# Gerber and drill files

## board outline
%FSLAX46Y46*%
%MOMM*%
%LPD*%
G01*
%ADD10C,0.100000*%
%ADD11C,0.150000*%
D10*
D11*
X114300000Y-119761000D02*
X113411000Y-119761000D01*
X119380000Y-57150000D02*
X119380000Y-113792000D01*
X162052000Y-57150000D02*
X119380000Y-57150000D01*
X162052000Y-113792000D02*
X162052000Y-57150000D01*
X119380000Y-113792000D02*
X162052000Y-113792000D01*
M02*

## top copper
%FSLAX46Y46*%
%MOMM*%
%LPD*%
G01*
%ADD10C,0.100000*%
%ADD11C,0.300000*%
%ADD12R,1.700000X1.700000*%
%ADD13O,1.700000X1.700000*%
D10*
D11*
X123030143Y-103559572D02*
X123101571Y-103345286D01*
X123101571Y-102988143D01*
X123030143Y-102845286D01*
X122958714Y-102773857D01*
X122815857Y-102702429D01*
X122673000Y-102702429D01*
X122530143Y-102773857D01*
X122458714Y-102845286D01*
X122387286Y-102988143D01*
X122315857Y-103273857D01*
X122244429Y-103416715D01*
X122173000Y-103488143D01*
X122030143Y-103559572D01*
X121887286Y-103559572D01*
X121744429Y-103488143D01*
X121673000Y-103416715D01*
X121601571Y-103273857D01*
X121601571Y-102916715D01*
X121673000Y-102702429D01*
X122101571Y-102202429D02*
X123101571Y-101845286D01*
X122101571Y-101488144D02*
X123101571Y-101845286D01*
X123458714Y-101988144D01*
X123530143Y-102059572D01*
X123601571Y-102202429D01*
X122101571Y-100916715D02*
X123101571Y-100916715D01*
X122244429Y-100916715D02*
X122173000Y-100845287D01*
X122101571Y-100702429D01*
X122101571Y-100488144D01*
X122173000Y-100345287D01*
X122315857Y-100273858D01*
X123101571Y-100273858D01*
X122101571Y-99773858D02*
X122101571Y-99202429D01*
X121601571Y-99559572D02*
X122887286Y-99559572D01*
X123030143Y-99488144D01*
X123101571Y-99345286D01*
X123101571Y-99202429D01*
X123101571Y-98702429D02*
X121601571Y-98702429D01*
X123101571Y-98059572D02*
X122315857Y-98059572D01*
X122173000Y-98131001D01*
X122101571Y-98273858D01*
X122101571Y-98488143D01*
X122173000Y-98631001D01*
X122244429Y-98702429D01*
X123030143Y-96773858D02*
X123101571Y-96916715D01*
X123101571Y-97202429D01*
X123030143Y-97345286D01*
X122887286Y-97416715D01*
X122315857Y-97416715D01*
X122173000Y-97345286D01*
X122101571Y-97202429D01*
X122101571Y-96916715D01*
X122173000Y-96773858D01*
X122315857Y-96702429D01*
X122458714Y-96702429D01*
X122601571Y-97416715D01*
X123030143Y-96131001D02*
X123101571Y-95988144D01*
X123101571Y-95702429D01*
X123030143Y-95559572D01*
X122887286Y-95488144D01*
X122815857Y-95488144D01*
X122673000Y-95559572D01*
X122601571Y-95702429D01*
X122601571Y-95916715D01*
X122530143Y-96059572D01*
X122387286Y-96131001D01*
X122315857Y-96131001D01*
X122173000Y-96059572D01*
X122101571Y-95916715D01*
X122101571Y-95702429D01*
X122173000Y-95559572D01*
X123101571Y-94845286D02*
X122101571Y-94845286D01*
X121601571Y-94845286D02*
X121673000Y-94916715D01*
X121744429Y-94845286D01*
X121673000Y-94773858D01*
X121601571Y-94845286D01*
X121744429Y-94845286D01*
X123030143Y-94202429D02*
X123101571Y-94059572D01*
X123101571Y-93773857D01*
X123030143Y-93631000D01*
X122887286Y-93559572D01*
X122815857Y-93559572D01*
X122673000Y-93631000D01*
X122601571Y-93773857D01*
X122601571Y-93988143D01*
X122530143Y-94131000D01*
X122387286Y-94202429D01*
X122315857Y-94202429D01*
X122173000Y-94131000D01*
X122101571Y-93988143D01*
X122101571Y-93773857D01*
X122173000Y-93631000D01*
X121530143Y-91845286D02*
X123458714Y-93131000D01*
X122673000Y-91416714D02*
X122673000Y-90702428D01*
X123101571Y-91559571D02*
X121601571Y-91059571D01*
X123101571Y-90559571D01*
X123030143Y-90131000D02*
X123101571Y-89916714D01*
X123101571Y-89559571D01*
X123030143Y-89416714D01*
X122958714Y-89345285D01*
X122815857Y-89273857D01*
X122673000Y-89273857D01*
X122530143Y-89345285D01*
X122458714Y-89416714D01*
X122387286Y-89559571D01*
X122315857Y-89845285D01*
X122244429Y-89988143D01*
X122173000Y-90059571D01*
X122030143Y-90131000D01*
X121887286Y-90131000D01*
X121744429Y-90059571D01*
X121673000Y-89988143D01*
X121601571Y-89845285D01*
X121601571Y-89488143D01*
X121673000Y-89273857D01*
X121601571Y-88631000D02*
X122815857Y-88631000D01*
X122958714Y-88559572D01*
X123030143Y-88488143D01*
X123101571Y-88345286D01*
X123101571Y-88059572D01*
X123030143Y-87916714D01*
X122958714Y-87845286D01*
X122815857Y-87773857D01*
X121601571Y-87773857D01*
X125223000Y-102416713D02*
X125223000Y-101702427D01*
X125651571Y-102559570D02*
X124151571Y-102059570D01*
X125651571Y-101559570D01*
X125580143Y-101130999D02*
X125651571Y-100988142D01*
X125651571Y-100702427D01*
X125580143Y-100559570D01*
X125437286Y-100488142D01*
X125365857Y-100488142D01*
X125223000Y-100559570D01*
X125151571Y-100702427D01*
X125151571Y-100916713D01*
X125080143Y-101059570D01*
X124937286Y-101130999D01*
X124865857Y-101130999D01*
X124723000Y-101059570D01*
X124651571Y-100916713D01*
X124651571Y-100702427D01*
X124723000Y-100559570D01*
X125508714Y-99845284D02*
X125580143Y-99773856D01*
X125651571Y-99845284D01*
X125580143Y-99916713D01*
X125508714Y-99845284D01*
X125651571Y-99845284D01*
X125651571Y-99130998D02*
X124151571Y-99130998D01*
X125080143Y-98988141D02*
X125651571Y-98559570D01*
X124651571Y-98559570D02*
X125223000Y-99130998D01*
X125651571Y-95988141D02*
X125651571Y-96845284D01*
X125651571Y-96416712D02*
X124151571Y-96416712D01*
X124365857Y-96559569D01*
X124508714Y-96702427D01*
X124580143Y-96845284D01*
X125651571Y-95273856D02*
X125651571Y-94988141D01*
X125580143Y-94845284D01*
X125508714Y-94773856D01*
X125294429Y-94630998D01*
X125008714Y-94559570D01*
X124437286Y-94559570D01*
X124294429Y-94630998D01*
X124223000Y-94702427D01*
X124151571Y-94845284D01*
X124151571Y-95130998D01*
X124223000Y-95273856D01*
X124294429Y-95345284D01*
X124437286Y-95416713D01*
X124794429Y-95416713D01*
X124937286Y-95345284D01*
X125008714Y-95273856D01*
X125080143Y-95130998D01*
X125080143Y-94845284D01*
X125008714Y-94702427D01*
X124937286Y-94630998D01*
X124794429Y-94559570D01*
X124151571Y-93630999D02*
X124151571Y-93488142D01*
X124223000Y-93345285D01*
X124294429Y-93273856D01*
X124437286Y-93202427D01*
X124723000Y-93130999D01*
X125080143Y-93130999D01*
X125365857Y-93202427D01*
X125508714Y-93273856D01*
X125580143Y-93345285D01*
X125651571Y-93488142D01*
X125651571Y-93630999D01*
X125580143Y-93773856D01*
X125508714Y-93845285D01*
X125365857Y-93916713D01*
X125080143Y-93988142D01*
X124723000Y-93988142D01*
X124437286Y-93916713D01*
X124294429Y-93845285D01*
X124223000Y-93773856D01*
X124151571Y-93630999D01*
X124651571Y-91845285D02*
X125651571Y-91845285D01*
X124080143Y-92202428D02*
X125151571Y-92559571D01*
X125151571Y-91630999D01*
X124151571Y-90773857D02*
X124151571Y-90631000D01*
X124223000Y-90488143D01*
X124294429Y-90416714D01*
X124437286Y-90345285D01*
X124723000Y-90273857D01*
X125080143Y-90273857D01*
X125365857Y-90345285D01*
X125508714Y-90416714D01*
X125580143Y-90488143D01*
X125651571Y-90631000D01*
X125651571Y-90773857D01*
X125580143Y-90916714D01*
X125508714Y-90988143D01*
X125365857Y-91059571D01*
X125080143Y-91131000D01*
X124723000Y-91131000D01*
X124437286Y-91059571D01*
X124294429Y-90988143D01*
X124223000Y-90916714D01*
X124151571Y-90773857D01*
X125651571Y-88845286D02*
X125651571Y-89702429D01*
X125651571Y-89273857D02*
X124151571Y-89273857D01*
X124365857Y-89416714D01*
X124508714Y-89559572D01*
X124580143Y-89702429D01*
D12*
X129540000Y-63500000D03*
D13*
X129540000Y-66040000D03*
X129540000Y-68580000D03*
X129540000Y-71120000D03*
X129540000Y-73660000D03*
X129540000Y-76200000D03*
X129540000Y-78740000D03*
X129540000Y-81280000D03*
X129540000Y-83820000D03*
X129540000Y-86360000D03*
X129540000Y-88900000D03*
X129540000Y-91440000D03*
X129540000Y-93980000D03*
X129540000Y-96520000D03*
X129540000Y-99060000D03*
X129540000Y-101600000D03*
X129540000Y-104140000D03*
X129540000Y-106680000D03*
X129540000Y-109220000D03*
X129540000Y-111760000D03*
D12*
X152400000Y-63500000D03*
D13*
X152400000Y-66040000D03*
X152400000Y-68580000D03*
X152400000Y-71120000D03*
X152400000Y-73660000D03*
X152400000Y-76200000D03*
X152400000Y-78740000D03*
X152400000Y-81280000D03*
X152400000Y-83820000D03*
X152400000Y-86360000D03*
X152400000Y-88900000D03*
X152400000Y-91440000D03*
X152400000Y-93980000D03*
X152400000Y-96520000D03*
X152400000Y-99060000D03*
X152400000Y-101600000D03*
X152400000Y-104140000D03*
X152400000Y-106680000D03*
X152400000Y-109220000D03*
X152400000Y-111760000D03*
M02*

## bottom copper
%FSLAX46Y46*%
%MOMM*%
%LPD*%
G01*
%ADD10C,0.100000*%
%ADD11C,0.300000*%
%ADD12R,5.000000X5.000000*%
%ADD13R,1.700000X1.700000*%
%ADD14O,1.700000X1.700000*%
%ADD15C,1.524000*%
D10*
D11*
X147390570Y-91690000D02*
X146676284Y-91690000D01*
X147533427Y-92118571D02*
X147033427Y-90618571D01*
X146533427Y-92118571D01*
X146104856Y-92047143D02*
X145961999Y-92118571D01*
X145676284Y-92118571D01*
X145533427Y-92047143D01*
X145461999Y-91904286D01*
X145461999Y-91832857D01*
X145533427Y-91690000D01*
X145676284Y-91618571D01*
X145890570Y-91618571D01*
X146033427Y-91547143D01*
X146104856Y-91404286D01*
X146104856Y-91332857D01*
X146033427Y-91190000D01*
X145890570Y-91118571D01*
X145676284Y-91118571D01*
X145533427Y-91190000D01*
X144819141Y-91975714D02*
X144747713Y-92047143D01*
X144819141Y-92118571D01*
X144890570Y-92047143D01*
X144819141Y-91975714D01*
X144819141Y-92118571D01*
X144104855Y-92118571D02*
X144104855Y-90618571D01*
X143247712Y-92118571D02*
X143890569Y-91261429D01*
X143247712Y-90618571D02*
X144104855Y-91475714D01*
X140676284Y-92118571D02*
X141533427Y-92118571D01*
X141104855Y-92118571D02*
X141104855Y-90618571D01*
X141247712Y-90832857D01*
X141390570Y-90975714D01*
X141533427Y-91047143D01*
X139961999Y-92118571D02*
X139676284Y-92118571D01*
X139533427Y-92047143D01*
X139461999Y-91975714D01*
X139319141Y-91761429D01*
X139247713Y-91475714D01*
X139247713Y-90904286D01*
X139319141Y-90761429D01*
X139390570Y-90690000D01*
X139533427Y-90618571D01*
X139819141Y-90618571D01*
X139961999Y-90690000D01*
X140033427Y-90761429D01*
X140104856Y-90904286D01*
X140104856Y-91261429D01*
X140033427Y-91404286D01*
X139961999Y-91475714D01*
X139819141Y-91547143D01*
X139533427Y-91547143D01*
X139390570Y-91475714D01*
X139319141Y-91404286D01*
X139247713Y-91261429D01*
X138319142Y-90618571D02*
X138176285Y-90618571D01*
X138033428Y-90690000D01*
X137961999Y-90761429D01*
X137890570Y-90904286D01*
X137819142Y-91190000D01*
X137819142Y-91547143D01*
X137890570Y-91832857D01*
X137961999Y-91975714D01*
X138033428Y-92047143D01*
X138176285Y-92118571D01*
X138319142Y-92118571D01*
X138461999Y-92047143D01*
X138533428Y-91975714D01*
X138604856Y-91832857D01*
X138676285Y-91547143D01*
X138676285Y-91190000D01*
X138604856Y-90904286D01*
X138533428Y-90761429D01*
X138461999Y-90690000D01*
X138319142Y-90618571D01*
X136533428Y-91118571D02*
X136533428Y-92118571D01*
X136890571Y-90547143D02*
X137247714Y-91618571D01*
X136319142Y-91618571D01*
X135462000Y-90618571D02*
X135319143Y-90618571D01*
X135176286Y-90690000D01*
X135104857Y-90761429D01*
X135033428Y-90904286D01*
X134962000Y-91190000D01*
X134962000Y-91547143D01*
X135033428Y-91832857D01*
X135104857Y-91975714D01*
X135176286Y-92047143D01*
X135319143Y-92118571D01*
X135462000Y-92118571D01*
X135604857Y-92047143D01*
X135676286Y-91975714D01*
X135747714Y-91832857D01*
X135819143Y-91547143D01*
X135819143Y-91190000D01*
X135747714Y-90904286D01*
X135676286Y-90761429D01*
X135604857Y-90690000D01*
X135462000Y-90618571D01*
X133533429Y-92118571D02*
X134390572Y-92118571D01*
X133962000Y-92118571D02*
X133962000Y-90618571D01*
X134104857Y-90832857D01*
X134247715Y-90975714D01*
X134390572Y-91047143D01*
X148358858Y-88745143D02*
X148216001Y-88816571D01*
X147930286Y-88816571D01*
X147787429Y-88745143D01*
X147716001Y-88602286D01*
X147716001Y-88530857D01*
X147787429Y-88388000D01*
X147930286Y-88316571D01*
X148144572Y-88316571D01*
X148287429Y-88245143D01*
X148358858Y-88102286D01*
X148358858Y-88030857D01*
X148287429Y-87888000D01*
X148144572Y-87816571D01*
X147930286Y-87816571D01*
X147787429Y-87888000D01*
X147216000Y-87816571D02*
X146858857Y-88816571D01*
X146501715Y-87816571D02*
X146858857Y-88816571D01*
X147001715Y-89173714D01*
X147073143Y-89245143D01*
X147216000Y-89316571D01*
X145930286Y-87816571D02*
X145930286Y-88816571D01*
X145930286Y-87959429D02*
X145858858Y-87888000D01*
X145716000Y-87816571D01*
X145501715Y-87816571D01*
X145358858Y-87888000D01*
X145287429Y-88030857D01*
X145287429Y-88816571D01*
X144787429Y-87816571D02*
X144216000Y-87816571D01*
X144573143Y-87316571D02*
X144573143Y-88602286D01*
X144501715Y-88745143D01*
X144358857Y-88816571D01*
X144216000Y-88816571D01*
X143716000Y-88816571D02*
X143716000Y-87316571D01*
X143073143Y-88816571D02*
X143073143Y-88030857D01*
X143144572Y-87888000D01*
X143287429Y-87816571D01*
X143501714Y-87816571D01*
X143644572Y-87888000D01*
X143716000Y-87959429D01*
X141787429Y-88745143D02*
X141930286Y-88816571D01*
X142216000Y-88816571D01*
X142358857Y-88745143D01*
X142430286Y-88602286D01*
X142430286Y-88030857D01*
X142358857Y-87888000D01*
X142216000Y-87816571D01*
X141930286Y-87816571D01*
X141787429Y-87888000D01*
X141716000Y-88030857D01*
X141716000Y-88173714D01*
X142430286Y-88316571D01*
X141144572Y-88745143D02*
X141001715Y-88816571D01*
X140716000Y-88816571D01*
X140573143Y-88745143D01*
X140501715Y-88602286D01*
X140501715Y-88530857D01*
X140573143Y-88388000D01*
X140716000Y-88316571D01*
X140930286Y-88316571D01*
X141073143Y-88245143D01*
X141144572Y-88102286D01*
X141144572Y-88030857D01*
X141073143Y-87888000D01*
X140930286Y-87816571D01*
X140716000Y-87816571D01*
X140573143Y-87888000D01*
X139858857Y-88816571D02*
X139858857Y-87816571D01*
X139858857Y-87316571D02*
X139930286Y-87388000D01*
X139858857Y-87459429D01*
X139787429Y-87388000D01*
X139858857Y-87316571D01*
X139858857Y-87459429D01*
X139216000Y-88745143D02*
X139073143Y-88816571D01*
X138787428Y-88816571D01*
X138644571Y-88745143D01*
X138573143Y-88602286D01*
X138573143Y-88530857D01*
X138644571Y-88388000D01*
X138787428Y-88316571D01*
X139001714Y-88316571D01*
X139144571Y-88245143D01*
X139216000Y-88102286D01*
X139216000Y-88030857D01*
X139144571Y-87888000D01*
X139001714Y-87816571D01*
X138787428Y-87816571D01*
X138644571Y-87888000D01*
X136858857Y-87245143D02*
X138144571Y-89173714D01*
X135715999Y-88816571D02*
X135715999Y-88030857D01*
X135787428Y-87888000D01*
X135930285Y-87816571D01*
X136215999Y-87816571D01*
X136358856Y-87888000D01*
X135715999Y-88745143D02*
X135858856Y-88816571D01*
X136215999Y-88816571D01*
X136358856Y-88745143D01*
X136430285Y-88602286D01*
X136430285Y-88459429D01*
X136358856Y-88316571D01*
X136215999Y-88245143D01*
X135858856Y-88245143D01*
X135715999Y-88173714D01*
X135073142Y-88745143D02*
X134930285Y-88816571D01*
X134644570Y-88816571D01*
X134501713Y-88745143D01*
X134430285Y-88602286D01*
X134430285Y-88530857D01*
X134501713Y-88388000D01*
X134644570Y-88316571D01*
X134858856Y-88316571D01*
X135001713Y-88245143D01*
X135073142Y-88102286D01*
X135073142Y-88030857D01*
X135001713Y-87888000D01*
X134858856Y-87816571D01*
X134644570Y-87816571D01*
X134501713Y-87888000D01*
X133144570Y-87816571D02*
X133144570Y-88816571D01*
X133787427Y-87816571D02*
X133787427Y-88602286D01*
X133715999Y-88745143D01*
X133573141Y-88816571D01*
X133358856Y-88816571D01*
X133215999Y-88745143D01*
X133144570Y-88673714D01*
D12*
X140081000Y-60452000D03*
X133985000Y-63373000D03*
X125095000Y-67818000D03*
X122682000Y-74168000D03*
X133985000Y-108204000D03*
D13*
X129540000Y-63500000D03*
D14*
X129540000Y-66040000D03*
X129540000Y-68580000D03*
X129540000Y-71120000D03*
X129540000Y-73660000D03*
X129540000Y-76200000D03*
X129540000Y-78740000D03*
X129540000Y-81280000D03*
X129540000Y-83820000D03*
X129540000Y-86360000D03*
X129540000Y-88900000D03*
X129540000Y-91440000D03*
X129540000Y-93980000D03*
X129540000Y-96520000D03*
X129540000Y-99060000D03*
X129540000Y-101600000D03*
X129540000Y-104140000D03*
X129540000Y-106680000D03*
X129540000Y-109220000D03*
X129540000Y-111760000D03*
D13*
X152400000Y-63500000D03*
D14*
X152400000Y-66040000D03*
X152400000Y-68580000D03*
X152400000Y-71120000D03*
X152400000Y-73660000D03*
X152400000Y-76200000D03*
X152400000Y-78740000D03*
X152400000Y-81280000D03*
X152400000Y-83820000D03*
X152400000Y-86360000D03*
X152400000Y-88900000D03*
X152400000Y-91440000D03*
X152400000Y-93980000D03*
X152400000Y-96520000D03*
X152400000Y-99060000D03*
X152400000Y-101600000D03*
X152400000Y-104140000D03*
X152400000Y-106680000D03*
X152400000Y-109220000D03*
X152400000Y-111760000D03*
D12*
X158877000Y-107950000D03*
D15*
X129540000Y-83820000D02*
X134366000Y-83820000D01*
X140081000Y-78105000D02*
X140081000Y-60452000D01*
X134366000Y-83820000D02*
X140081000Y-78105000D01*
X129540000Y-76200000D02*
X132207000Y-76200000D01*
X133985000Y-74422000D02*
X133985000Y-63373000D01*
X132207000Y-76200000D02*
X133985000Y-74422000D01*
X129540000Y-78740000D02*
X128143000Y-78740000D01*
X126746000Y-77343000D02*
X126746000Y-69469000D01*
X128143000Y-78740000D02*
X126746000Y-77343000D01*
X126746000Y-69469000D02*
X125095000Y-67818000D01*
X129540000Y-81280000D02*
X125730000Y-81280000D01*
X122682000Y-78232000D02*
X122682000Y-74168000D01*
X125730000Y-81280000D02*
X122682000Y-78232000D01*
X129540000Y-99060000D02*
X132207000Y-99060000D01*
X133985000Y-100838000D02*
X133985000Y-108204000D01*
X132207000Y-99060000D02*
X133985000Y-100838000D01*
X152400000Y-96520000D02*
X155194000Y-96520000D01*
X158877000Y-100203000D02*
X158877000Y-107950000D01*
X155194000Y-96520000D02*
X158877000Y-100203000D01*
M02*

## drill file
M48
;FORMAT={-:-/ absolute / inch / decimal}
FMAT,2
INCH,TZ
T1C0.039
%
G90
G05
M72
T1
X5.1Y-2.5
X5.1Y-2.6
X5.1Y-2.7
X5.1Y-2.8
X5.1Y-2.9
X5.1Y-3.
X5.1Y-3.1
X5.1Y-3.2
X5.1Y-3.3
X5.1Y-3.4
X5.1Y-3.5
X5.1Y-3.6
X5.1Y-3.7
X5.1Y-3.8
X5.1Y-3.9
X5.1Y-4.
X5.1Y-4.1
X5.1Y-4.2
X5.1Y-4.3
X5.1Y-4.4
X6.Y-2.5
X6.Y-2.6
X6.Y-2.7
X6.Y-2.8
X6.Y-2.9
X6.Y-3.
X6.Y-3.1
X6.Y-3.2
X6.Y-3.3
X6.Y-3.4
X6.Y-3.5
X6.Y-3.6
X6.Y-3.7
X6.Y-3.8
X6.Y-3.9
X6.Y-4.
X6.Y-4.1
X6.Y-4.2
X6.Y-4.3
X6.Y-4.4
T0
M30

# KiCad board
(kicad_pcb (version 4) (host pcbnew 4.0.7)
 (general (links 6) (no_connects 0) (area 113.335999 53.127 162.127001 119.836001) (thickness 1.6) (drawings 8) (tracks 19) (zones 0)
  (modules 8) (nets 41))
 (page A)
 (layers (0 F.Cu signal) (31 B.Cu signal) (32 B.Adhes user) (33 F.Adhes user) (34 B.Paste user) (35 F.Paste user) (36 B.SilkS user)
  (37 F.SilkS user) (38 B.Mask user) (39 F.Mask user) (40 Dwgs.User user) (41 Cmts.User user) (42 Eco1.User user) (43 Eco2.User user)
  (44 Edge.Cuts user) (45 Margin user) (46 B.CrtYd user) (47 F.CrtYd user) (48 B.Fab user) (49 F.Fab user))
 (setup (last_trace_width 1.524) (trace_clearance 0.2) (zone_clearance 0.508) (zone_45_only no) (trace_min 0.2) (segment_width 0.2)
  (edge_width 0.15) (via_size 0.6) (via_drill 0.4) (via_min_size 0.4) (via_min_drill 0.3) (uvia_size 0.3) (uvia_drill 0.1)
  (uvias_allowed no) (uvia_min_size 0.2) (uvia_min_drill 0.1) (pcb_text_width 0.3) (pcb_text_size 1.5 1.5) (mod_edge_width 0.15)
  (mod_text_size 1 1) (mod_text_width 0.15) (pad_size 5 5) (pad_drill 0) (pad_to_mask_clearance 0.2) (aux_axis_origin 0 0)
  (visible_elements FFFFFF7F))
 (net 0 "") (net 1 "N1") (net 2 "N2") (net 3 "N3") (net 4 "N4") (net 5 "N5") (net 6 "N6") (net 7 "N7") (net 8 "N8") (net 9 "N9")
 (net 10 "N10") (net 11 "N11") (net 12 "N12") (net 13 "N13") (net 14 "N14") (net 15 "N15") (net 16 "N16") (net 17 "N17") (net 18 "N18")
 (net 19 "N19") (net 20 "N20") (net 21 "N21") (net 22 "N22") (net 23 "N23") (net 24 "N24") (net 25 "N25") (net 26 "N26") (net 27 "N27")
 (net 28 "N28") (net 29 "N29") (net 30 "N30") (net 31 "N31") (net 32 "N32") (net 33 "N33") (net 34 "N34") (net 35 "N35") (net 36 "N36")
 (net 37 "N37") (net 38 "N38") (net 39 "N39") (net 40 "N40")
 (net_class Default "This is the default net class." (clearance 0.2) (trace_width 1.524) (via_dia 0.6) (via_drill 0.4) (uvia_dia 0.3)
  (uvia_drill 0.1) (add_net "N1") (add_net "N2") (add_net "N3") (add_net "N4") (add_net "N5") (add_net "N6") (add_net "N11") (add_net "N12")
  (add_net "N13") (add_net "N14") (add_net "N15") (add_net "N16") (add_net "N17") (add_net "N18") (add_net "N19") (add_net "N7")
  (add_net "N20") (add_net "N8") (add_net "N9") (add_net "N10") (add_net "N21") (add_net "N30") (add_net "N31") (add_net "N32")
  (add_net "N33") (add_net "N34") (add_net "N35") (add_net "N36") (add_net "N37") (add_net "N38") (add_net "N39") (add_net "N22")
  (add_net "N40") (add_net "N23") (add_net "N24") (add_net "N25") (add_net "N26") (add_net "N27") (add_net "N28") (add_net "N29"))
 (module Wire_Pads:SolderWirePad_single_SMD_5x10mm (layer B.Cu) (at 140.081 60.452)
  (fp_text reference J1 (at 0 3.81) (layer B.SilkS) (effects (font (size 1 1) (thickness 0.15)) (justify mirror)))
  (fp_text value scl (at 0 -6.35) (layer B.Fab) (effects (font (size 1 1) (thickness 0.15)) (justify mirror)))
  (pad 1 smd rect (at 0 0) (size 5 5) (layers B.Cu B.Paste B.Mask) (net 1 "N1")))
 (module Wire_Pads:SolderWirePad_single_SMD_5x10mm (layer B.Cu) (at 133.985 63.373)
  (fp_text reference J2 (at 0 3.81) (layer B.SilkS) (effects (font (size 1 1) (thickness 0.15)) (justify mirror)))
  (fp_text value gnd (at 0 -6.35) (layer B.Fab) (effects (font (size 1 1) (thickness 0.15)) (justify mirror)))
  (pad 1 smd rect (at 0 0) (size 5 5) (layers B.Cu B.Paste B.Mask) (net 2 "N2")))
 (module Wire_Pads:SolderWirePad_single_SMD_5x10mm (layer B.Cu) (at 125.095 67.818)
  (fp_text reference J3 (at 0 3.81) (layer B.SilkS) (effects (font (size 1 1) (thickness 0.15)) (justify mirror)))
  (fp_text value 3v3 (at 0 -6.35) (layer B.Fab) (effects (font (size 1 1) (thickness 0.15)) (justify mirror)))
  (pad 1 smd rect (at 0 0) (size 5 5) (layers B.Cu B.Paste B.Mask) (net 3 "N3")))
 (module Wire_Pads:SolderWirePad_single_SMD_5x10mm (layer B.Cu) (at 122.682 74.168)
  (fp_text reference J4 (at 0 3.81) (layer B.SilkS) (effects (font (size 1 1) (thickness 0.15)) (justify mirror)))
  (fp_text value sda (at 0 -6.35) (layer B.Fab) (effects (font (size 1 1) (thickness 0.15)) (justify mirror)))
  (pad 1 smd rect (at 0 0) (size 5 5) (layers B.Cu B.Paste B.Mask) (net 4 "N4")))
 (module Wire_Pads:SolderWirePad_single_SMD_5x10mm (layer B.Cu) (at 133.985 108.204)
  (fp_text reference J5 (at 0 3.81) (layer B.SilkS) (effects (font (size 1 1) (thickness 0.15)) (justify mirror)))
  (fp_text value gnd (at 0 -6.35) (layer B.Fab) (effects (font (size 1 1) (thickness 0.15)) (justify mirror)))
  (pad 1 smd rect (at 0 0) (size 5 5) (layers B.Cu B.Paste B.Mask) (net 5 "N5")))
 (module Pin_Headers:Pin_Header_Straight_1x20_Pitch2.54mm (layer F.Cu) (at 129.54 63.5)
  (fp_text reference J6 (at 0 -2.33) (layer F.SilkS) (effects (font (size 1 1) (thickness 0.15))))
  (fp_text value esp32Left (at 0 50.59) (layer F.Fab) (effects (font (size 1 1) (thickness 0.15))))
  (pad 1 thru_hole rect (at 0 0) (size 1.7 1.7) (drill 1) (layers *.Cu *.Mask) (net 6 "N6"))
  (pad 2 thru_hole oval (at 0 2.54) (size 1.7 1.7) (drill 1) (layers *.Cu *.Mask) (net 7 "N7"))
  (pad 3 thru_hole oval (at 0 5.08) (size 1.7 1.7) (drill 1) (layers *.Cu *.Mask) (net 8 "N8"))
  (pad 4 thru_hole oval (at 0 7.62) (size 1.7 1.7) (drill 1) (layers *.Cu *.Mask) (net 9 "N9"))
  (pad 5 thru_hole oval (at 0 10.16) (size 1.7 1.7) (drill 1) (layers *.Cu *.Mask) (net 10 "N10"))
  (pad 6 thru_hole oval (at 0 12.7) (size 1.7 1.7) (drill 1) (layers *.Cu *.Mask) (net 2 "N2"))
  (pad 7 thru_hole oval (at 0 15.24) (size 1.7 1.7) (drill 1) (layers *.Cu *.Mask) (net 3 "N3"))
  (pad 8 thru_hole oval (at 0 17.78) (size 1.7 1.7) (drill 1) (layers *.Cu *.Mask) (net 4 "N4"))
  (pad 9 thru_hole oval (at 0 20.32) (size 1.7 1.7) (drill 1) (layers *.Cu *.Mask) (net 1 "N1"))
  (pad 10 thru_hole oval (at 0 22.86) (size 1.7 1.7) (drill 1) (layers *.Cu *.Mask) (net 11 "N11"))
  (pad 11 thru_hole oval (at 0 25.4) (size 1.7 1.7) (drill 1) (layers *.Cu *.Mask) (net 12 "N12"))
  (pad 12 thru_hole oval (at 0 27.94) (size 1.7 1.7) (drill 1) (layers *.Cu *.Mask) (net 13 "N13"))
  (pad 13 thru_hole oval (at 0 30.48) (size 1.7 1.7) (drill 1) (layers *.Cu *.Mask) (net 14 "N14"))
  (pad 14 thru_hole oval (at 0 33.02) (size 1.7 1.7) (drill 1) (layers *.Cu *.Mask) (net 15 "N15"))
  (pad 15 thru_hole oval (at 0 35.56) (size 1.7 1.7) (drill 1) (layers *.Cu *.Mask) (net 5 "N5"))
  (pad 16 thru_hole oval (at 0 38.1) (size 1.7 1.7) (drill 1) (layers *.Cu *.Mask) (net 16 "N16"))
  (pad 17 thru_hole oval (at 0 40.64) (size 1.7 1.7) (drill 1) (layers *.Cu *.Mask) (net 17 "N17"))
  (pad 18 thru_hole oval (at 0 43.18) (size 1.7 1.7) (drill 1) (layers *.Cu *.Mask) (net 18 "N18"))
  (pad 19 thru_hole oval (at 0 45.72) (size 1.7 1.7) (drill 1) (layers *.Cu *.Mask) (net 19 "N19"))
  (pad 20 thru_hole oval (at 0 48.26) (size 1.7 1.7) (drill 1) (layers *.Cu *.Mask) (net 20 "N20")))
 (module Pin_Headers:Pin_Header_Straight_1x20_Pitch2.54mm (layer F.Cu) (at 152.4 63.5)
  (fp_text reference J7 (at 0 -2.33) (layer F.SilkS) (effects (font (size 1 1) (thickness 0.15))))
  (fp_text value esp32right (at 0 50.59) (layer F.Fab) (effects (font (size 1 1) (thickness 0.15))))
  (pad 1 thru_hole rect (at 0 0) (size 1.7 1.7) (drill 1) (layers *.Cu *.Mask) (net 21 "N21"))
  (pad 2 thru_hole oval (at 0 2.54) (size 1.7 1.7) (drill 1) (layers *.Cu *.Mask) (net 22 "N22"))
  (pad 3 thru_hole oval (at 0 5.08) (size 1.7 1.7) (drill 1) (layers *.Cu *.Mask) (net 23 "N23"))
  (pad 4 thru_hole oval (at 0 7.62) (size 1.7 1.7) (drill 1) (layers *.Cu *.Mask) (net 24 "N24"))
  (pad 5 thru_hole oval (at 0 10.16) (size 1.7 1.7) (drill 1) (layers *.Cu *.Mask) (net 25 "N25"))
  (pad 6 thru_hole oval (at 0 12.7) (size 1.7 1.7) (drill 1) (layers *.Cu *.Mask) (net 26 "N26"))
  (pad 7 thru_hole oval (at 0 15.24) (size 1.7 1.7) (drill 1) (layers *.Cu *.Mask) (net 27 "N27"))
  (pad 8 thru_hole oval (at 0 17.78) (size 1.7 1.7) (drill 1) (layers *.Cu *.Mask) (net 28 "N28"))
  (pad 9 thru_hole oval (at 0 20.32) (size 1.7 1.7) (drill 1) (layers *.Cu *.Mask) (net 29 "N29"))
  (pad 10 thru_hole oval (at 0 22.86) (size 1.7 1.7) (drill 1) (layers *.Cu *.Mask) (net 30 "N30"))
  (pad 11 thru_hole oval (at 0 25.4) (size 1.7 1.7) (drill 1) (layers *.Cu *.Mask) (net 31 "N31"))
  (pad 12 thru_hole oval (at 0 27.94) (size 1.7 1.7) (drill 1) (layers *.Cu *.Mask) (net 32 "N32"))
  (pad 13 thru_hole oval (at 0 30.48) (size 1.7 1.7) (drill 1) (layers *.Cu *.Mask) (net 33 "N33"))
  (pad 14 thru_hole oval (at 0 33.02) (size 1.7 1.7) (drill 1) (layers *.Cu *.Mask) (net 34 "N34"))
  (pad 15 thru_hole oval (at 0 35.56) (size 1.7 1.7) (drill 1) (layers *.Cu *.Mask) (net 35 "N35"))
  (pad 16 thru_hole oval (at 0 38.1) (size 1.7 1.7) (drill 1) (layers *.Cu *.Mask) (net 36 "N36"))
  (pad 17 thru_hole oval (at 0 40.64) (size 1.7 1.7) (drill 1) (layers *.Cu *.Mask) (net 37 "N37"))
  (pad 18 thru_hole oval (at 0 43.18) (size 1.7 1.7) (drill 1) (layers *.Cu *.Mask) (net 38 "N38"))
  (pad 19 thru_hole oval (at 0 45.72) (size 1.7 1.7) (drill 1) (layers *.Cu *.Mask) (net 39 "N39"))
  (pad 20 thru_hole oval (at 0 48.26) (size 1.7 1.7) (drill 1) (layers *.Cu *.Mask) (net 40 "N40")))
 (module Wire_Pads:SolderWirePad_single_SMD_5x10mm (layer B.Cu) (at 158.877 107.95)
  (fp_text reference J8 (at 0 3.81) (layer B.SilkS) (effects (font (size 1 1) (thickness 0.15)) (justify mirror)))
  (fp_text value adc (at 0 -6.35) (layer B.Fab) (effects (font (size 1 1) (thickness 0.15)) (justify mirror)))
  (pad 1 smd rect (at 0 0) (size 5 5) (layers B.Cu B.Paste B.Mask) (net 34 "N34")))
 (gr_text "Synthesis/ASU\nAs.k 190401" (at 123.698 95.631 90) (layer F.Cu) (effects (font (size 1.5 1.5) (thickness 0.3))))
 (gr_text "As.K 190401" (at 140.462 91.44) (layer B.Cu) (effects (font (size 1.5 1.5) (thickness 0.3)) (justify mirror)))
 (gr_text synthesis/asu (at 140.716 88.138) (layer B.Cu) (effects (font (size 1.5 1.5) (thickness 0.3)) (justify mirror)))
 (gr_line (start 114.3 119.761) (end 113.411 119.761) (angle 90) (layer Edge.Cuts) (width 0.15))
 (gr_line (start 119.38 57.15) (end 119.38 113.792) (angle 90) (layer Edge.Cuts) (width 0.15))
 (gr_line (start 162.052 57.15) (end 119.38 57.15) (angle 90) (layer Edge.Cuts) (width 0.15))
 (gr_line (start 162.052 113.792) (end 162.052 57.15) (angle 90) (layer Edge.Cuts) (width 0.15))
 (gr_line (start 119.38 113.792) (end 162.052 113.792) (angle 90) (layer Edge.Cuts) (width 0.15))
 (segment (start 129.54 83.82) (end 134.366 83.82) (width 1.524) (layer B.Cu) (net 1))
 (segment (start 140.081 78.105) (end 140.081 60.452) (width 1.524) (layer B.Cu) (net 1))
 (segment (start 134.366 83.82) (end 140.081 78.105) (width 1.524) (layer B.Cu) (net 1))
 (segment (start 129.54 76.2) (end 132.207 76.2) (width 1.524) (layer B.Cu) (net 2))
 (segment (start 133.985 74.422) (end 133.985 63.373) (width 1.524) (layer B.Cu) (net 2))
 (segment (start 132.207 76.2) (end 133.985 74.422) (width 1.524) (layer B.Cu) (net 2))
 (segment (start 129.54 78.74) (end 128.143 78.74) (width 1.524) (layer B.Cu) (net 3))
 (segment (start 126.746 77.343) (end 126.746 69.469) (width 1.524) (layer B.Cu) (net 3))
 (segment (start 128.143 78.74) (end 126.746 77.343) (width 1.524) (layer B.Cu) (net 3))
 (segment (start 126.746 69.469) (end 125.095 67.818) (width 1.524) (layer B.Cu) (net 3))
 (segment (start 129.54 81.28) (end 125.73 81.28) (width 1.524) (layer B.Cu) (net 4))
 (segment (start 122.682 78.232) (end 122.682 74.168) (width 1.524) (layer B.Cu) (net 4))
 (segment (start 125.73 81.28) (end 122.682 78.232) (width 1.524) (layer B.Cu) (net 4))
 (segment (start 129.54 99.06) (end 132.207 99.06) (width 1.524) (layer B.Cu) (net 5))
 (segment (start 133.985 100.838) (end 133.985 108.204) (width 1.524) (layer B.Cu) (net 5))
 (segment (start 132.207 99.06) (end 133.985 100.838) (width 1.524) (layer B.Cu) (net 5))
 (segment (start 152.4 96.52) (end 155.194 96.52) (width 1.524) (layer B.Cu) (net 34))
 (segment (start 158.877 100.203) (end 158.877 107.95) (width 1.524) (layer B.Cu) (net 34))
 (segment (start 155.194 96.52) (end 158.877 100.203) (width 1.524) (layer B.Cu) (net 34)))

